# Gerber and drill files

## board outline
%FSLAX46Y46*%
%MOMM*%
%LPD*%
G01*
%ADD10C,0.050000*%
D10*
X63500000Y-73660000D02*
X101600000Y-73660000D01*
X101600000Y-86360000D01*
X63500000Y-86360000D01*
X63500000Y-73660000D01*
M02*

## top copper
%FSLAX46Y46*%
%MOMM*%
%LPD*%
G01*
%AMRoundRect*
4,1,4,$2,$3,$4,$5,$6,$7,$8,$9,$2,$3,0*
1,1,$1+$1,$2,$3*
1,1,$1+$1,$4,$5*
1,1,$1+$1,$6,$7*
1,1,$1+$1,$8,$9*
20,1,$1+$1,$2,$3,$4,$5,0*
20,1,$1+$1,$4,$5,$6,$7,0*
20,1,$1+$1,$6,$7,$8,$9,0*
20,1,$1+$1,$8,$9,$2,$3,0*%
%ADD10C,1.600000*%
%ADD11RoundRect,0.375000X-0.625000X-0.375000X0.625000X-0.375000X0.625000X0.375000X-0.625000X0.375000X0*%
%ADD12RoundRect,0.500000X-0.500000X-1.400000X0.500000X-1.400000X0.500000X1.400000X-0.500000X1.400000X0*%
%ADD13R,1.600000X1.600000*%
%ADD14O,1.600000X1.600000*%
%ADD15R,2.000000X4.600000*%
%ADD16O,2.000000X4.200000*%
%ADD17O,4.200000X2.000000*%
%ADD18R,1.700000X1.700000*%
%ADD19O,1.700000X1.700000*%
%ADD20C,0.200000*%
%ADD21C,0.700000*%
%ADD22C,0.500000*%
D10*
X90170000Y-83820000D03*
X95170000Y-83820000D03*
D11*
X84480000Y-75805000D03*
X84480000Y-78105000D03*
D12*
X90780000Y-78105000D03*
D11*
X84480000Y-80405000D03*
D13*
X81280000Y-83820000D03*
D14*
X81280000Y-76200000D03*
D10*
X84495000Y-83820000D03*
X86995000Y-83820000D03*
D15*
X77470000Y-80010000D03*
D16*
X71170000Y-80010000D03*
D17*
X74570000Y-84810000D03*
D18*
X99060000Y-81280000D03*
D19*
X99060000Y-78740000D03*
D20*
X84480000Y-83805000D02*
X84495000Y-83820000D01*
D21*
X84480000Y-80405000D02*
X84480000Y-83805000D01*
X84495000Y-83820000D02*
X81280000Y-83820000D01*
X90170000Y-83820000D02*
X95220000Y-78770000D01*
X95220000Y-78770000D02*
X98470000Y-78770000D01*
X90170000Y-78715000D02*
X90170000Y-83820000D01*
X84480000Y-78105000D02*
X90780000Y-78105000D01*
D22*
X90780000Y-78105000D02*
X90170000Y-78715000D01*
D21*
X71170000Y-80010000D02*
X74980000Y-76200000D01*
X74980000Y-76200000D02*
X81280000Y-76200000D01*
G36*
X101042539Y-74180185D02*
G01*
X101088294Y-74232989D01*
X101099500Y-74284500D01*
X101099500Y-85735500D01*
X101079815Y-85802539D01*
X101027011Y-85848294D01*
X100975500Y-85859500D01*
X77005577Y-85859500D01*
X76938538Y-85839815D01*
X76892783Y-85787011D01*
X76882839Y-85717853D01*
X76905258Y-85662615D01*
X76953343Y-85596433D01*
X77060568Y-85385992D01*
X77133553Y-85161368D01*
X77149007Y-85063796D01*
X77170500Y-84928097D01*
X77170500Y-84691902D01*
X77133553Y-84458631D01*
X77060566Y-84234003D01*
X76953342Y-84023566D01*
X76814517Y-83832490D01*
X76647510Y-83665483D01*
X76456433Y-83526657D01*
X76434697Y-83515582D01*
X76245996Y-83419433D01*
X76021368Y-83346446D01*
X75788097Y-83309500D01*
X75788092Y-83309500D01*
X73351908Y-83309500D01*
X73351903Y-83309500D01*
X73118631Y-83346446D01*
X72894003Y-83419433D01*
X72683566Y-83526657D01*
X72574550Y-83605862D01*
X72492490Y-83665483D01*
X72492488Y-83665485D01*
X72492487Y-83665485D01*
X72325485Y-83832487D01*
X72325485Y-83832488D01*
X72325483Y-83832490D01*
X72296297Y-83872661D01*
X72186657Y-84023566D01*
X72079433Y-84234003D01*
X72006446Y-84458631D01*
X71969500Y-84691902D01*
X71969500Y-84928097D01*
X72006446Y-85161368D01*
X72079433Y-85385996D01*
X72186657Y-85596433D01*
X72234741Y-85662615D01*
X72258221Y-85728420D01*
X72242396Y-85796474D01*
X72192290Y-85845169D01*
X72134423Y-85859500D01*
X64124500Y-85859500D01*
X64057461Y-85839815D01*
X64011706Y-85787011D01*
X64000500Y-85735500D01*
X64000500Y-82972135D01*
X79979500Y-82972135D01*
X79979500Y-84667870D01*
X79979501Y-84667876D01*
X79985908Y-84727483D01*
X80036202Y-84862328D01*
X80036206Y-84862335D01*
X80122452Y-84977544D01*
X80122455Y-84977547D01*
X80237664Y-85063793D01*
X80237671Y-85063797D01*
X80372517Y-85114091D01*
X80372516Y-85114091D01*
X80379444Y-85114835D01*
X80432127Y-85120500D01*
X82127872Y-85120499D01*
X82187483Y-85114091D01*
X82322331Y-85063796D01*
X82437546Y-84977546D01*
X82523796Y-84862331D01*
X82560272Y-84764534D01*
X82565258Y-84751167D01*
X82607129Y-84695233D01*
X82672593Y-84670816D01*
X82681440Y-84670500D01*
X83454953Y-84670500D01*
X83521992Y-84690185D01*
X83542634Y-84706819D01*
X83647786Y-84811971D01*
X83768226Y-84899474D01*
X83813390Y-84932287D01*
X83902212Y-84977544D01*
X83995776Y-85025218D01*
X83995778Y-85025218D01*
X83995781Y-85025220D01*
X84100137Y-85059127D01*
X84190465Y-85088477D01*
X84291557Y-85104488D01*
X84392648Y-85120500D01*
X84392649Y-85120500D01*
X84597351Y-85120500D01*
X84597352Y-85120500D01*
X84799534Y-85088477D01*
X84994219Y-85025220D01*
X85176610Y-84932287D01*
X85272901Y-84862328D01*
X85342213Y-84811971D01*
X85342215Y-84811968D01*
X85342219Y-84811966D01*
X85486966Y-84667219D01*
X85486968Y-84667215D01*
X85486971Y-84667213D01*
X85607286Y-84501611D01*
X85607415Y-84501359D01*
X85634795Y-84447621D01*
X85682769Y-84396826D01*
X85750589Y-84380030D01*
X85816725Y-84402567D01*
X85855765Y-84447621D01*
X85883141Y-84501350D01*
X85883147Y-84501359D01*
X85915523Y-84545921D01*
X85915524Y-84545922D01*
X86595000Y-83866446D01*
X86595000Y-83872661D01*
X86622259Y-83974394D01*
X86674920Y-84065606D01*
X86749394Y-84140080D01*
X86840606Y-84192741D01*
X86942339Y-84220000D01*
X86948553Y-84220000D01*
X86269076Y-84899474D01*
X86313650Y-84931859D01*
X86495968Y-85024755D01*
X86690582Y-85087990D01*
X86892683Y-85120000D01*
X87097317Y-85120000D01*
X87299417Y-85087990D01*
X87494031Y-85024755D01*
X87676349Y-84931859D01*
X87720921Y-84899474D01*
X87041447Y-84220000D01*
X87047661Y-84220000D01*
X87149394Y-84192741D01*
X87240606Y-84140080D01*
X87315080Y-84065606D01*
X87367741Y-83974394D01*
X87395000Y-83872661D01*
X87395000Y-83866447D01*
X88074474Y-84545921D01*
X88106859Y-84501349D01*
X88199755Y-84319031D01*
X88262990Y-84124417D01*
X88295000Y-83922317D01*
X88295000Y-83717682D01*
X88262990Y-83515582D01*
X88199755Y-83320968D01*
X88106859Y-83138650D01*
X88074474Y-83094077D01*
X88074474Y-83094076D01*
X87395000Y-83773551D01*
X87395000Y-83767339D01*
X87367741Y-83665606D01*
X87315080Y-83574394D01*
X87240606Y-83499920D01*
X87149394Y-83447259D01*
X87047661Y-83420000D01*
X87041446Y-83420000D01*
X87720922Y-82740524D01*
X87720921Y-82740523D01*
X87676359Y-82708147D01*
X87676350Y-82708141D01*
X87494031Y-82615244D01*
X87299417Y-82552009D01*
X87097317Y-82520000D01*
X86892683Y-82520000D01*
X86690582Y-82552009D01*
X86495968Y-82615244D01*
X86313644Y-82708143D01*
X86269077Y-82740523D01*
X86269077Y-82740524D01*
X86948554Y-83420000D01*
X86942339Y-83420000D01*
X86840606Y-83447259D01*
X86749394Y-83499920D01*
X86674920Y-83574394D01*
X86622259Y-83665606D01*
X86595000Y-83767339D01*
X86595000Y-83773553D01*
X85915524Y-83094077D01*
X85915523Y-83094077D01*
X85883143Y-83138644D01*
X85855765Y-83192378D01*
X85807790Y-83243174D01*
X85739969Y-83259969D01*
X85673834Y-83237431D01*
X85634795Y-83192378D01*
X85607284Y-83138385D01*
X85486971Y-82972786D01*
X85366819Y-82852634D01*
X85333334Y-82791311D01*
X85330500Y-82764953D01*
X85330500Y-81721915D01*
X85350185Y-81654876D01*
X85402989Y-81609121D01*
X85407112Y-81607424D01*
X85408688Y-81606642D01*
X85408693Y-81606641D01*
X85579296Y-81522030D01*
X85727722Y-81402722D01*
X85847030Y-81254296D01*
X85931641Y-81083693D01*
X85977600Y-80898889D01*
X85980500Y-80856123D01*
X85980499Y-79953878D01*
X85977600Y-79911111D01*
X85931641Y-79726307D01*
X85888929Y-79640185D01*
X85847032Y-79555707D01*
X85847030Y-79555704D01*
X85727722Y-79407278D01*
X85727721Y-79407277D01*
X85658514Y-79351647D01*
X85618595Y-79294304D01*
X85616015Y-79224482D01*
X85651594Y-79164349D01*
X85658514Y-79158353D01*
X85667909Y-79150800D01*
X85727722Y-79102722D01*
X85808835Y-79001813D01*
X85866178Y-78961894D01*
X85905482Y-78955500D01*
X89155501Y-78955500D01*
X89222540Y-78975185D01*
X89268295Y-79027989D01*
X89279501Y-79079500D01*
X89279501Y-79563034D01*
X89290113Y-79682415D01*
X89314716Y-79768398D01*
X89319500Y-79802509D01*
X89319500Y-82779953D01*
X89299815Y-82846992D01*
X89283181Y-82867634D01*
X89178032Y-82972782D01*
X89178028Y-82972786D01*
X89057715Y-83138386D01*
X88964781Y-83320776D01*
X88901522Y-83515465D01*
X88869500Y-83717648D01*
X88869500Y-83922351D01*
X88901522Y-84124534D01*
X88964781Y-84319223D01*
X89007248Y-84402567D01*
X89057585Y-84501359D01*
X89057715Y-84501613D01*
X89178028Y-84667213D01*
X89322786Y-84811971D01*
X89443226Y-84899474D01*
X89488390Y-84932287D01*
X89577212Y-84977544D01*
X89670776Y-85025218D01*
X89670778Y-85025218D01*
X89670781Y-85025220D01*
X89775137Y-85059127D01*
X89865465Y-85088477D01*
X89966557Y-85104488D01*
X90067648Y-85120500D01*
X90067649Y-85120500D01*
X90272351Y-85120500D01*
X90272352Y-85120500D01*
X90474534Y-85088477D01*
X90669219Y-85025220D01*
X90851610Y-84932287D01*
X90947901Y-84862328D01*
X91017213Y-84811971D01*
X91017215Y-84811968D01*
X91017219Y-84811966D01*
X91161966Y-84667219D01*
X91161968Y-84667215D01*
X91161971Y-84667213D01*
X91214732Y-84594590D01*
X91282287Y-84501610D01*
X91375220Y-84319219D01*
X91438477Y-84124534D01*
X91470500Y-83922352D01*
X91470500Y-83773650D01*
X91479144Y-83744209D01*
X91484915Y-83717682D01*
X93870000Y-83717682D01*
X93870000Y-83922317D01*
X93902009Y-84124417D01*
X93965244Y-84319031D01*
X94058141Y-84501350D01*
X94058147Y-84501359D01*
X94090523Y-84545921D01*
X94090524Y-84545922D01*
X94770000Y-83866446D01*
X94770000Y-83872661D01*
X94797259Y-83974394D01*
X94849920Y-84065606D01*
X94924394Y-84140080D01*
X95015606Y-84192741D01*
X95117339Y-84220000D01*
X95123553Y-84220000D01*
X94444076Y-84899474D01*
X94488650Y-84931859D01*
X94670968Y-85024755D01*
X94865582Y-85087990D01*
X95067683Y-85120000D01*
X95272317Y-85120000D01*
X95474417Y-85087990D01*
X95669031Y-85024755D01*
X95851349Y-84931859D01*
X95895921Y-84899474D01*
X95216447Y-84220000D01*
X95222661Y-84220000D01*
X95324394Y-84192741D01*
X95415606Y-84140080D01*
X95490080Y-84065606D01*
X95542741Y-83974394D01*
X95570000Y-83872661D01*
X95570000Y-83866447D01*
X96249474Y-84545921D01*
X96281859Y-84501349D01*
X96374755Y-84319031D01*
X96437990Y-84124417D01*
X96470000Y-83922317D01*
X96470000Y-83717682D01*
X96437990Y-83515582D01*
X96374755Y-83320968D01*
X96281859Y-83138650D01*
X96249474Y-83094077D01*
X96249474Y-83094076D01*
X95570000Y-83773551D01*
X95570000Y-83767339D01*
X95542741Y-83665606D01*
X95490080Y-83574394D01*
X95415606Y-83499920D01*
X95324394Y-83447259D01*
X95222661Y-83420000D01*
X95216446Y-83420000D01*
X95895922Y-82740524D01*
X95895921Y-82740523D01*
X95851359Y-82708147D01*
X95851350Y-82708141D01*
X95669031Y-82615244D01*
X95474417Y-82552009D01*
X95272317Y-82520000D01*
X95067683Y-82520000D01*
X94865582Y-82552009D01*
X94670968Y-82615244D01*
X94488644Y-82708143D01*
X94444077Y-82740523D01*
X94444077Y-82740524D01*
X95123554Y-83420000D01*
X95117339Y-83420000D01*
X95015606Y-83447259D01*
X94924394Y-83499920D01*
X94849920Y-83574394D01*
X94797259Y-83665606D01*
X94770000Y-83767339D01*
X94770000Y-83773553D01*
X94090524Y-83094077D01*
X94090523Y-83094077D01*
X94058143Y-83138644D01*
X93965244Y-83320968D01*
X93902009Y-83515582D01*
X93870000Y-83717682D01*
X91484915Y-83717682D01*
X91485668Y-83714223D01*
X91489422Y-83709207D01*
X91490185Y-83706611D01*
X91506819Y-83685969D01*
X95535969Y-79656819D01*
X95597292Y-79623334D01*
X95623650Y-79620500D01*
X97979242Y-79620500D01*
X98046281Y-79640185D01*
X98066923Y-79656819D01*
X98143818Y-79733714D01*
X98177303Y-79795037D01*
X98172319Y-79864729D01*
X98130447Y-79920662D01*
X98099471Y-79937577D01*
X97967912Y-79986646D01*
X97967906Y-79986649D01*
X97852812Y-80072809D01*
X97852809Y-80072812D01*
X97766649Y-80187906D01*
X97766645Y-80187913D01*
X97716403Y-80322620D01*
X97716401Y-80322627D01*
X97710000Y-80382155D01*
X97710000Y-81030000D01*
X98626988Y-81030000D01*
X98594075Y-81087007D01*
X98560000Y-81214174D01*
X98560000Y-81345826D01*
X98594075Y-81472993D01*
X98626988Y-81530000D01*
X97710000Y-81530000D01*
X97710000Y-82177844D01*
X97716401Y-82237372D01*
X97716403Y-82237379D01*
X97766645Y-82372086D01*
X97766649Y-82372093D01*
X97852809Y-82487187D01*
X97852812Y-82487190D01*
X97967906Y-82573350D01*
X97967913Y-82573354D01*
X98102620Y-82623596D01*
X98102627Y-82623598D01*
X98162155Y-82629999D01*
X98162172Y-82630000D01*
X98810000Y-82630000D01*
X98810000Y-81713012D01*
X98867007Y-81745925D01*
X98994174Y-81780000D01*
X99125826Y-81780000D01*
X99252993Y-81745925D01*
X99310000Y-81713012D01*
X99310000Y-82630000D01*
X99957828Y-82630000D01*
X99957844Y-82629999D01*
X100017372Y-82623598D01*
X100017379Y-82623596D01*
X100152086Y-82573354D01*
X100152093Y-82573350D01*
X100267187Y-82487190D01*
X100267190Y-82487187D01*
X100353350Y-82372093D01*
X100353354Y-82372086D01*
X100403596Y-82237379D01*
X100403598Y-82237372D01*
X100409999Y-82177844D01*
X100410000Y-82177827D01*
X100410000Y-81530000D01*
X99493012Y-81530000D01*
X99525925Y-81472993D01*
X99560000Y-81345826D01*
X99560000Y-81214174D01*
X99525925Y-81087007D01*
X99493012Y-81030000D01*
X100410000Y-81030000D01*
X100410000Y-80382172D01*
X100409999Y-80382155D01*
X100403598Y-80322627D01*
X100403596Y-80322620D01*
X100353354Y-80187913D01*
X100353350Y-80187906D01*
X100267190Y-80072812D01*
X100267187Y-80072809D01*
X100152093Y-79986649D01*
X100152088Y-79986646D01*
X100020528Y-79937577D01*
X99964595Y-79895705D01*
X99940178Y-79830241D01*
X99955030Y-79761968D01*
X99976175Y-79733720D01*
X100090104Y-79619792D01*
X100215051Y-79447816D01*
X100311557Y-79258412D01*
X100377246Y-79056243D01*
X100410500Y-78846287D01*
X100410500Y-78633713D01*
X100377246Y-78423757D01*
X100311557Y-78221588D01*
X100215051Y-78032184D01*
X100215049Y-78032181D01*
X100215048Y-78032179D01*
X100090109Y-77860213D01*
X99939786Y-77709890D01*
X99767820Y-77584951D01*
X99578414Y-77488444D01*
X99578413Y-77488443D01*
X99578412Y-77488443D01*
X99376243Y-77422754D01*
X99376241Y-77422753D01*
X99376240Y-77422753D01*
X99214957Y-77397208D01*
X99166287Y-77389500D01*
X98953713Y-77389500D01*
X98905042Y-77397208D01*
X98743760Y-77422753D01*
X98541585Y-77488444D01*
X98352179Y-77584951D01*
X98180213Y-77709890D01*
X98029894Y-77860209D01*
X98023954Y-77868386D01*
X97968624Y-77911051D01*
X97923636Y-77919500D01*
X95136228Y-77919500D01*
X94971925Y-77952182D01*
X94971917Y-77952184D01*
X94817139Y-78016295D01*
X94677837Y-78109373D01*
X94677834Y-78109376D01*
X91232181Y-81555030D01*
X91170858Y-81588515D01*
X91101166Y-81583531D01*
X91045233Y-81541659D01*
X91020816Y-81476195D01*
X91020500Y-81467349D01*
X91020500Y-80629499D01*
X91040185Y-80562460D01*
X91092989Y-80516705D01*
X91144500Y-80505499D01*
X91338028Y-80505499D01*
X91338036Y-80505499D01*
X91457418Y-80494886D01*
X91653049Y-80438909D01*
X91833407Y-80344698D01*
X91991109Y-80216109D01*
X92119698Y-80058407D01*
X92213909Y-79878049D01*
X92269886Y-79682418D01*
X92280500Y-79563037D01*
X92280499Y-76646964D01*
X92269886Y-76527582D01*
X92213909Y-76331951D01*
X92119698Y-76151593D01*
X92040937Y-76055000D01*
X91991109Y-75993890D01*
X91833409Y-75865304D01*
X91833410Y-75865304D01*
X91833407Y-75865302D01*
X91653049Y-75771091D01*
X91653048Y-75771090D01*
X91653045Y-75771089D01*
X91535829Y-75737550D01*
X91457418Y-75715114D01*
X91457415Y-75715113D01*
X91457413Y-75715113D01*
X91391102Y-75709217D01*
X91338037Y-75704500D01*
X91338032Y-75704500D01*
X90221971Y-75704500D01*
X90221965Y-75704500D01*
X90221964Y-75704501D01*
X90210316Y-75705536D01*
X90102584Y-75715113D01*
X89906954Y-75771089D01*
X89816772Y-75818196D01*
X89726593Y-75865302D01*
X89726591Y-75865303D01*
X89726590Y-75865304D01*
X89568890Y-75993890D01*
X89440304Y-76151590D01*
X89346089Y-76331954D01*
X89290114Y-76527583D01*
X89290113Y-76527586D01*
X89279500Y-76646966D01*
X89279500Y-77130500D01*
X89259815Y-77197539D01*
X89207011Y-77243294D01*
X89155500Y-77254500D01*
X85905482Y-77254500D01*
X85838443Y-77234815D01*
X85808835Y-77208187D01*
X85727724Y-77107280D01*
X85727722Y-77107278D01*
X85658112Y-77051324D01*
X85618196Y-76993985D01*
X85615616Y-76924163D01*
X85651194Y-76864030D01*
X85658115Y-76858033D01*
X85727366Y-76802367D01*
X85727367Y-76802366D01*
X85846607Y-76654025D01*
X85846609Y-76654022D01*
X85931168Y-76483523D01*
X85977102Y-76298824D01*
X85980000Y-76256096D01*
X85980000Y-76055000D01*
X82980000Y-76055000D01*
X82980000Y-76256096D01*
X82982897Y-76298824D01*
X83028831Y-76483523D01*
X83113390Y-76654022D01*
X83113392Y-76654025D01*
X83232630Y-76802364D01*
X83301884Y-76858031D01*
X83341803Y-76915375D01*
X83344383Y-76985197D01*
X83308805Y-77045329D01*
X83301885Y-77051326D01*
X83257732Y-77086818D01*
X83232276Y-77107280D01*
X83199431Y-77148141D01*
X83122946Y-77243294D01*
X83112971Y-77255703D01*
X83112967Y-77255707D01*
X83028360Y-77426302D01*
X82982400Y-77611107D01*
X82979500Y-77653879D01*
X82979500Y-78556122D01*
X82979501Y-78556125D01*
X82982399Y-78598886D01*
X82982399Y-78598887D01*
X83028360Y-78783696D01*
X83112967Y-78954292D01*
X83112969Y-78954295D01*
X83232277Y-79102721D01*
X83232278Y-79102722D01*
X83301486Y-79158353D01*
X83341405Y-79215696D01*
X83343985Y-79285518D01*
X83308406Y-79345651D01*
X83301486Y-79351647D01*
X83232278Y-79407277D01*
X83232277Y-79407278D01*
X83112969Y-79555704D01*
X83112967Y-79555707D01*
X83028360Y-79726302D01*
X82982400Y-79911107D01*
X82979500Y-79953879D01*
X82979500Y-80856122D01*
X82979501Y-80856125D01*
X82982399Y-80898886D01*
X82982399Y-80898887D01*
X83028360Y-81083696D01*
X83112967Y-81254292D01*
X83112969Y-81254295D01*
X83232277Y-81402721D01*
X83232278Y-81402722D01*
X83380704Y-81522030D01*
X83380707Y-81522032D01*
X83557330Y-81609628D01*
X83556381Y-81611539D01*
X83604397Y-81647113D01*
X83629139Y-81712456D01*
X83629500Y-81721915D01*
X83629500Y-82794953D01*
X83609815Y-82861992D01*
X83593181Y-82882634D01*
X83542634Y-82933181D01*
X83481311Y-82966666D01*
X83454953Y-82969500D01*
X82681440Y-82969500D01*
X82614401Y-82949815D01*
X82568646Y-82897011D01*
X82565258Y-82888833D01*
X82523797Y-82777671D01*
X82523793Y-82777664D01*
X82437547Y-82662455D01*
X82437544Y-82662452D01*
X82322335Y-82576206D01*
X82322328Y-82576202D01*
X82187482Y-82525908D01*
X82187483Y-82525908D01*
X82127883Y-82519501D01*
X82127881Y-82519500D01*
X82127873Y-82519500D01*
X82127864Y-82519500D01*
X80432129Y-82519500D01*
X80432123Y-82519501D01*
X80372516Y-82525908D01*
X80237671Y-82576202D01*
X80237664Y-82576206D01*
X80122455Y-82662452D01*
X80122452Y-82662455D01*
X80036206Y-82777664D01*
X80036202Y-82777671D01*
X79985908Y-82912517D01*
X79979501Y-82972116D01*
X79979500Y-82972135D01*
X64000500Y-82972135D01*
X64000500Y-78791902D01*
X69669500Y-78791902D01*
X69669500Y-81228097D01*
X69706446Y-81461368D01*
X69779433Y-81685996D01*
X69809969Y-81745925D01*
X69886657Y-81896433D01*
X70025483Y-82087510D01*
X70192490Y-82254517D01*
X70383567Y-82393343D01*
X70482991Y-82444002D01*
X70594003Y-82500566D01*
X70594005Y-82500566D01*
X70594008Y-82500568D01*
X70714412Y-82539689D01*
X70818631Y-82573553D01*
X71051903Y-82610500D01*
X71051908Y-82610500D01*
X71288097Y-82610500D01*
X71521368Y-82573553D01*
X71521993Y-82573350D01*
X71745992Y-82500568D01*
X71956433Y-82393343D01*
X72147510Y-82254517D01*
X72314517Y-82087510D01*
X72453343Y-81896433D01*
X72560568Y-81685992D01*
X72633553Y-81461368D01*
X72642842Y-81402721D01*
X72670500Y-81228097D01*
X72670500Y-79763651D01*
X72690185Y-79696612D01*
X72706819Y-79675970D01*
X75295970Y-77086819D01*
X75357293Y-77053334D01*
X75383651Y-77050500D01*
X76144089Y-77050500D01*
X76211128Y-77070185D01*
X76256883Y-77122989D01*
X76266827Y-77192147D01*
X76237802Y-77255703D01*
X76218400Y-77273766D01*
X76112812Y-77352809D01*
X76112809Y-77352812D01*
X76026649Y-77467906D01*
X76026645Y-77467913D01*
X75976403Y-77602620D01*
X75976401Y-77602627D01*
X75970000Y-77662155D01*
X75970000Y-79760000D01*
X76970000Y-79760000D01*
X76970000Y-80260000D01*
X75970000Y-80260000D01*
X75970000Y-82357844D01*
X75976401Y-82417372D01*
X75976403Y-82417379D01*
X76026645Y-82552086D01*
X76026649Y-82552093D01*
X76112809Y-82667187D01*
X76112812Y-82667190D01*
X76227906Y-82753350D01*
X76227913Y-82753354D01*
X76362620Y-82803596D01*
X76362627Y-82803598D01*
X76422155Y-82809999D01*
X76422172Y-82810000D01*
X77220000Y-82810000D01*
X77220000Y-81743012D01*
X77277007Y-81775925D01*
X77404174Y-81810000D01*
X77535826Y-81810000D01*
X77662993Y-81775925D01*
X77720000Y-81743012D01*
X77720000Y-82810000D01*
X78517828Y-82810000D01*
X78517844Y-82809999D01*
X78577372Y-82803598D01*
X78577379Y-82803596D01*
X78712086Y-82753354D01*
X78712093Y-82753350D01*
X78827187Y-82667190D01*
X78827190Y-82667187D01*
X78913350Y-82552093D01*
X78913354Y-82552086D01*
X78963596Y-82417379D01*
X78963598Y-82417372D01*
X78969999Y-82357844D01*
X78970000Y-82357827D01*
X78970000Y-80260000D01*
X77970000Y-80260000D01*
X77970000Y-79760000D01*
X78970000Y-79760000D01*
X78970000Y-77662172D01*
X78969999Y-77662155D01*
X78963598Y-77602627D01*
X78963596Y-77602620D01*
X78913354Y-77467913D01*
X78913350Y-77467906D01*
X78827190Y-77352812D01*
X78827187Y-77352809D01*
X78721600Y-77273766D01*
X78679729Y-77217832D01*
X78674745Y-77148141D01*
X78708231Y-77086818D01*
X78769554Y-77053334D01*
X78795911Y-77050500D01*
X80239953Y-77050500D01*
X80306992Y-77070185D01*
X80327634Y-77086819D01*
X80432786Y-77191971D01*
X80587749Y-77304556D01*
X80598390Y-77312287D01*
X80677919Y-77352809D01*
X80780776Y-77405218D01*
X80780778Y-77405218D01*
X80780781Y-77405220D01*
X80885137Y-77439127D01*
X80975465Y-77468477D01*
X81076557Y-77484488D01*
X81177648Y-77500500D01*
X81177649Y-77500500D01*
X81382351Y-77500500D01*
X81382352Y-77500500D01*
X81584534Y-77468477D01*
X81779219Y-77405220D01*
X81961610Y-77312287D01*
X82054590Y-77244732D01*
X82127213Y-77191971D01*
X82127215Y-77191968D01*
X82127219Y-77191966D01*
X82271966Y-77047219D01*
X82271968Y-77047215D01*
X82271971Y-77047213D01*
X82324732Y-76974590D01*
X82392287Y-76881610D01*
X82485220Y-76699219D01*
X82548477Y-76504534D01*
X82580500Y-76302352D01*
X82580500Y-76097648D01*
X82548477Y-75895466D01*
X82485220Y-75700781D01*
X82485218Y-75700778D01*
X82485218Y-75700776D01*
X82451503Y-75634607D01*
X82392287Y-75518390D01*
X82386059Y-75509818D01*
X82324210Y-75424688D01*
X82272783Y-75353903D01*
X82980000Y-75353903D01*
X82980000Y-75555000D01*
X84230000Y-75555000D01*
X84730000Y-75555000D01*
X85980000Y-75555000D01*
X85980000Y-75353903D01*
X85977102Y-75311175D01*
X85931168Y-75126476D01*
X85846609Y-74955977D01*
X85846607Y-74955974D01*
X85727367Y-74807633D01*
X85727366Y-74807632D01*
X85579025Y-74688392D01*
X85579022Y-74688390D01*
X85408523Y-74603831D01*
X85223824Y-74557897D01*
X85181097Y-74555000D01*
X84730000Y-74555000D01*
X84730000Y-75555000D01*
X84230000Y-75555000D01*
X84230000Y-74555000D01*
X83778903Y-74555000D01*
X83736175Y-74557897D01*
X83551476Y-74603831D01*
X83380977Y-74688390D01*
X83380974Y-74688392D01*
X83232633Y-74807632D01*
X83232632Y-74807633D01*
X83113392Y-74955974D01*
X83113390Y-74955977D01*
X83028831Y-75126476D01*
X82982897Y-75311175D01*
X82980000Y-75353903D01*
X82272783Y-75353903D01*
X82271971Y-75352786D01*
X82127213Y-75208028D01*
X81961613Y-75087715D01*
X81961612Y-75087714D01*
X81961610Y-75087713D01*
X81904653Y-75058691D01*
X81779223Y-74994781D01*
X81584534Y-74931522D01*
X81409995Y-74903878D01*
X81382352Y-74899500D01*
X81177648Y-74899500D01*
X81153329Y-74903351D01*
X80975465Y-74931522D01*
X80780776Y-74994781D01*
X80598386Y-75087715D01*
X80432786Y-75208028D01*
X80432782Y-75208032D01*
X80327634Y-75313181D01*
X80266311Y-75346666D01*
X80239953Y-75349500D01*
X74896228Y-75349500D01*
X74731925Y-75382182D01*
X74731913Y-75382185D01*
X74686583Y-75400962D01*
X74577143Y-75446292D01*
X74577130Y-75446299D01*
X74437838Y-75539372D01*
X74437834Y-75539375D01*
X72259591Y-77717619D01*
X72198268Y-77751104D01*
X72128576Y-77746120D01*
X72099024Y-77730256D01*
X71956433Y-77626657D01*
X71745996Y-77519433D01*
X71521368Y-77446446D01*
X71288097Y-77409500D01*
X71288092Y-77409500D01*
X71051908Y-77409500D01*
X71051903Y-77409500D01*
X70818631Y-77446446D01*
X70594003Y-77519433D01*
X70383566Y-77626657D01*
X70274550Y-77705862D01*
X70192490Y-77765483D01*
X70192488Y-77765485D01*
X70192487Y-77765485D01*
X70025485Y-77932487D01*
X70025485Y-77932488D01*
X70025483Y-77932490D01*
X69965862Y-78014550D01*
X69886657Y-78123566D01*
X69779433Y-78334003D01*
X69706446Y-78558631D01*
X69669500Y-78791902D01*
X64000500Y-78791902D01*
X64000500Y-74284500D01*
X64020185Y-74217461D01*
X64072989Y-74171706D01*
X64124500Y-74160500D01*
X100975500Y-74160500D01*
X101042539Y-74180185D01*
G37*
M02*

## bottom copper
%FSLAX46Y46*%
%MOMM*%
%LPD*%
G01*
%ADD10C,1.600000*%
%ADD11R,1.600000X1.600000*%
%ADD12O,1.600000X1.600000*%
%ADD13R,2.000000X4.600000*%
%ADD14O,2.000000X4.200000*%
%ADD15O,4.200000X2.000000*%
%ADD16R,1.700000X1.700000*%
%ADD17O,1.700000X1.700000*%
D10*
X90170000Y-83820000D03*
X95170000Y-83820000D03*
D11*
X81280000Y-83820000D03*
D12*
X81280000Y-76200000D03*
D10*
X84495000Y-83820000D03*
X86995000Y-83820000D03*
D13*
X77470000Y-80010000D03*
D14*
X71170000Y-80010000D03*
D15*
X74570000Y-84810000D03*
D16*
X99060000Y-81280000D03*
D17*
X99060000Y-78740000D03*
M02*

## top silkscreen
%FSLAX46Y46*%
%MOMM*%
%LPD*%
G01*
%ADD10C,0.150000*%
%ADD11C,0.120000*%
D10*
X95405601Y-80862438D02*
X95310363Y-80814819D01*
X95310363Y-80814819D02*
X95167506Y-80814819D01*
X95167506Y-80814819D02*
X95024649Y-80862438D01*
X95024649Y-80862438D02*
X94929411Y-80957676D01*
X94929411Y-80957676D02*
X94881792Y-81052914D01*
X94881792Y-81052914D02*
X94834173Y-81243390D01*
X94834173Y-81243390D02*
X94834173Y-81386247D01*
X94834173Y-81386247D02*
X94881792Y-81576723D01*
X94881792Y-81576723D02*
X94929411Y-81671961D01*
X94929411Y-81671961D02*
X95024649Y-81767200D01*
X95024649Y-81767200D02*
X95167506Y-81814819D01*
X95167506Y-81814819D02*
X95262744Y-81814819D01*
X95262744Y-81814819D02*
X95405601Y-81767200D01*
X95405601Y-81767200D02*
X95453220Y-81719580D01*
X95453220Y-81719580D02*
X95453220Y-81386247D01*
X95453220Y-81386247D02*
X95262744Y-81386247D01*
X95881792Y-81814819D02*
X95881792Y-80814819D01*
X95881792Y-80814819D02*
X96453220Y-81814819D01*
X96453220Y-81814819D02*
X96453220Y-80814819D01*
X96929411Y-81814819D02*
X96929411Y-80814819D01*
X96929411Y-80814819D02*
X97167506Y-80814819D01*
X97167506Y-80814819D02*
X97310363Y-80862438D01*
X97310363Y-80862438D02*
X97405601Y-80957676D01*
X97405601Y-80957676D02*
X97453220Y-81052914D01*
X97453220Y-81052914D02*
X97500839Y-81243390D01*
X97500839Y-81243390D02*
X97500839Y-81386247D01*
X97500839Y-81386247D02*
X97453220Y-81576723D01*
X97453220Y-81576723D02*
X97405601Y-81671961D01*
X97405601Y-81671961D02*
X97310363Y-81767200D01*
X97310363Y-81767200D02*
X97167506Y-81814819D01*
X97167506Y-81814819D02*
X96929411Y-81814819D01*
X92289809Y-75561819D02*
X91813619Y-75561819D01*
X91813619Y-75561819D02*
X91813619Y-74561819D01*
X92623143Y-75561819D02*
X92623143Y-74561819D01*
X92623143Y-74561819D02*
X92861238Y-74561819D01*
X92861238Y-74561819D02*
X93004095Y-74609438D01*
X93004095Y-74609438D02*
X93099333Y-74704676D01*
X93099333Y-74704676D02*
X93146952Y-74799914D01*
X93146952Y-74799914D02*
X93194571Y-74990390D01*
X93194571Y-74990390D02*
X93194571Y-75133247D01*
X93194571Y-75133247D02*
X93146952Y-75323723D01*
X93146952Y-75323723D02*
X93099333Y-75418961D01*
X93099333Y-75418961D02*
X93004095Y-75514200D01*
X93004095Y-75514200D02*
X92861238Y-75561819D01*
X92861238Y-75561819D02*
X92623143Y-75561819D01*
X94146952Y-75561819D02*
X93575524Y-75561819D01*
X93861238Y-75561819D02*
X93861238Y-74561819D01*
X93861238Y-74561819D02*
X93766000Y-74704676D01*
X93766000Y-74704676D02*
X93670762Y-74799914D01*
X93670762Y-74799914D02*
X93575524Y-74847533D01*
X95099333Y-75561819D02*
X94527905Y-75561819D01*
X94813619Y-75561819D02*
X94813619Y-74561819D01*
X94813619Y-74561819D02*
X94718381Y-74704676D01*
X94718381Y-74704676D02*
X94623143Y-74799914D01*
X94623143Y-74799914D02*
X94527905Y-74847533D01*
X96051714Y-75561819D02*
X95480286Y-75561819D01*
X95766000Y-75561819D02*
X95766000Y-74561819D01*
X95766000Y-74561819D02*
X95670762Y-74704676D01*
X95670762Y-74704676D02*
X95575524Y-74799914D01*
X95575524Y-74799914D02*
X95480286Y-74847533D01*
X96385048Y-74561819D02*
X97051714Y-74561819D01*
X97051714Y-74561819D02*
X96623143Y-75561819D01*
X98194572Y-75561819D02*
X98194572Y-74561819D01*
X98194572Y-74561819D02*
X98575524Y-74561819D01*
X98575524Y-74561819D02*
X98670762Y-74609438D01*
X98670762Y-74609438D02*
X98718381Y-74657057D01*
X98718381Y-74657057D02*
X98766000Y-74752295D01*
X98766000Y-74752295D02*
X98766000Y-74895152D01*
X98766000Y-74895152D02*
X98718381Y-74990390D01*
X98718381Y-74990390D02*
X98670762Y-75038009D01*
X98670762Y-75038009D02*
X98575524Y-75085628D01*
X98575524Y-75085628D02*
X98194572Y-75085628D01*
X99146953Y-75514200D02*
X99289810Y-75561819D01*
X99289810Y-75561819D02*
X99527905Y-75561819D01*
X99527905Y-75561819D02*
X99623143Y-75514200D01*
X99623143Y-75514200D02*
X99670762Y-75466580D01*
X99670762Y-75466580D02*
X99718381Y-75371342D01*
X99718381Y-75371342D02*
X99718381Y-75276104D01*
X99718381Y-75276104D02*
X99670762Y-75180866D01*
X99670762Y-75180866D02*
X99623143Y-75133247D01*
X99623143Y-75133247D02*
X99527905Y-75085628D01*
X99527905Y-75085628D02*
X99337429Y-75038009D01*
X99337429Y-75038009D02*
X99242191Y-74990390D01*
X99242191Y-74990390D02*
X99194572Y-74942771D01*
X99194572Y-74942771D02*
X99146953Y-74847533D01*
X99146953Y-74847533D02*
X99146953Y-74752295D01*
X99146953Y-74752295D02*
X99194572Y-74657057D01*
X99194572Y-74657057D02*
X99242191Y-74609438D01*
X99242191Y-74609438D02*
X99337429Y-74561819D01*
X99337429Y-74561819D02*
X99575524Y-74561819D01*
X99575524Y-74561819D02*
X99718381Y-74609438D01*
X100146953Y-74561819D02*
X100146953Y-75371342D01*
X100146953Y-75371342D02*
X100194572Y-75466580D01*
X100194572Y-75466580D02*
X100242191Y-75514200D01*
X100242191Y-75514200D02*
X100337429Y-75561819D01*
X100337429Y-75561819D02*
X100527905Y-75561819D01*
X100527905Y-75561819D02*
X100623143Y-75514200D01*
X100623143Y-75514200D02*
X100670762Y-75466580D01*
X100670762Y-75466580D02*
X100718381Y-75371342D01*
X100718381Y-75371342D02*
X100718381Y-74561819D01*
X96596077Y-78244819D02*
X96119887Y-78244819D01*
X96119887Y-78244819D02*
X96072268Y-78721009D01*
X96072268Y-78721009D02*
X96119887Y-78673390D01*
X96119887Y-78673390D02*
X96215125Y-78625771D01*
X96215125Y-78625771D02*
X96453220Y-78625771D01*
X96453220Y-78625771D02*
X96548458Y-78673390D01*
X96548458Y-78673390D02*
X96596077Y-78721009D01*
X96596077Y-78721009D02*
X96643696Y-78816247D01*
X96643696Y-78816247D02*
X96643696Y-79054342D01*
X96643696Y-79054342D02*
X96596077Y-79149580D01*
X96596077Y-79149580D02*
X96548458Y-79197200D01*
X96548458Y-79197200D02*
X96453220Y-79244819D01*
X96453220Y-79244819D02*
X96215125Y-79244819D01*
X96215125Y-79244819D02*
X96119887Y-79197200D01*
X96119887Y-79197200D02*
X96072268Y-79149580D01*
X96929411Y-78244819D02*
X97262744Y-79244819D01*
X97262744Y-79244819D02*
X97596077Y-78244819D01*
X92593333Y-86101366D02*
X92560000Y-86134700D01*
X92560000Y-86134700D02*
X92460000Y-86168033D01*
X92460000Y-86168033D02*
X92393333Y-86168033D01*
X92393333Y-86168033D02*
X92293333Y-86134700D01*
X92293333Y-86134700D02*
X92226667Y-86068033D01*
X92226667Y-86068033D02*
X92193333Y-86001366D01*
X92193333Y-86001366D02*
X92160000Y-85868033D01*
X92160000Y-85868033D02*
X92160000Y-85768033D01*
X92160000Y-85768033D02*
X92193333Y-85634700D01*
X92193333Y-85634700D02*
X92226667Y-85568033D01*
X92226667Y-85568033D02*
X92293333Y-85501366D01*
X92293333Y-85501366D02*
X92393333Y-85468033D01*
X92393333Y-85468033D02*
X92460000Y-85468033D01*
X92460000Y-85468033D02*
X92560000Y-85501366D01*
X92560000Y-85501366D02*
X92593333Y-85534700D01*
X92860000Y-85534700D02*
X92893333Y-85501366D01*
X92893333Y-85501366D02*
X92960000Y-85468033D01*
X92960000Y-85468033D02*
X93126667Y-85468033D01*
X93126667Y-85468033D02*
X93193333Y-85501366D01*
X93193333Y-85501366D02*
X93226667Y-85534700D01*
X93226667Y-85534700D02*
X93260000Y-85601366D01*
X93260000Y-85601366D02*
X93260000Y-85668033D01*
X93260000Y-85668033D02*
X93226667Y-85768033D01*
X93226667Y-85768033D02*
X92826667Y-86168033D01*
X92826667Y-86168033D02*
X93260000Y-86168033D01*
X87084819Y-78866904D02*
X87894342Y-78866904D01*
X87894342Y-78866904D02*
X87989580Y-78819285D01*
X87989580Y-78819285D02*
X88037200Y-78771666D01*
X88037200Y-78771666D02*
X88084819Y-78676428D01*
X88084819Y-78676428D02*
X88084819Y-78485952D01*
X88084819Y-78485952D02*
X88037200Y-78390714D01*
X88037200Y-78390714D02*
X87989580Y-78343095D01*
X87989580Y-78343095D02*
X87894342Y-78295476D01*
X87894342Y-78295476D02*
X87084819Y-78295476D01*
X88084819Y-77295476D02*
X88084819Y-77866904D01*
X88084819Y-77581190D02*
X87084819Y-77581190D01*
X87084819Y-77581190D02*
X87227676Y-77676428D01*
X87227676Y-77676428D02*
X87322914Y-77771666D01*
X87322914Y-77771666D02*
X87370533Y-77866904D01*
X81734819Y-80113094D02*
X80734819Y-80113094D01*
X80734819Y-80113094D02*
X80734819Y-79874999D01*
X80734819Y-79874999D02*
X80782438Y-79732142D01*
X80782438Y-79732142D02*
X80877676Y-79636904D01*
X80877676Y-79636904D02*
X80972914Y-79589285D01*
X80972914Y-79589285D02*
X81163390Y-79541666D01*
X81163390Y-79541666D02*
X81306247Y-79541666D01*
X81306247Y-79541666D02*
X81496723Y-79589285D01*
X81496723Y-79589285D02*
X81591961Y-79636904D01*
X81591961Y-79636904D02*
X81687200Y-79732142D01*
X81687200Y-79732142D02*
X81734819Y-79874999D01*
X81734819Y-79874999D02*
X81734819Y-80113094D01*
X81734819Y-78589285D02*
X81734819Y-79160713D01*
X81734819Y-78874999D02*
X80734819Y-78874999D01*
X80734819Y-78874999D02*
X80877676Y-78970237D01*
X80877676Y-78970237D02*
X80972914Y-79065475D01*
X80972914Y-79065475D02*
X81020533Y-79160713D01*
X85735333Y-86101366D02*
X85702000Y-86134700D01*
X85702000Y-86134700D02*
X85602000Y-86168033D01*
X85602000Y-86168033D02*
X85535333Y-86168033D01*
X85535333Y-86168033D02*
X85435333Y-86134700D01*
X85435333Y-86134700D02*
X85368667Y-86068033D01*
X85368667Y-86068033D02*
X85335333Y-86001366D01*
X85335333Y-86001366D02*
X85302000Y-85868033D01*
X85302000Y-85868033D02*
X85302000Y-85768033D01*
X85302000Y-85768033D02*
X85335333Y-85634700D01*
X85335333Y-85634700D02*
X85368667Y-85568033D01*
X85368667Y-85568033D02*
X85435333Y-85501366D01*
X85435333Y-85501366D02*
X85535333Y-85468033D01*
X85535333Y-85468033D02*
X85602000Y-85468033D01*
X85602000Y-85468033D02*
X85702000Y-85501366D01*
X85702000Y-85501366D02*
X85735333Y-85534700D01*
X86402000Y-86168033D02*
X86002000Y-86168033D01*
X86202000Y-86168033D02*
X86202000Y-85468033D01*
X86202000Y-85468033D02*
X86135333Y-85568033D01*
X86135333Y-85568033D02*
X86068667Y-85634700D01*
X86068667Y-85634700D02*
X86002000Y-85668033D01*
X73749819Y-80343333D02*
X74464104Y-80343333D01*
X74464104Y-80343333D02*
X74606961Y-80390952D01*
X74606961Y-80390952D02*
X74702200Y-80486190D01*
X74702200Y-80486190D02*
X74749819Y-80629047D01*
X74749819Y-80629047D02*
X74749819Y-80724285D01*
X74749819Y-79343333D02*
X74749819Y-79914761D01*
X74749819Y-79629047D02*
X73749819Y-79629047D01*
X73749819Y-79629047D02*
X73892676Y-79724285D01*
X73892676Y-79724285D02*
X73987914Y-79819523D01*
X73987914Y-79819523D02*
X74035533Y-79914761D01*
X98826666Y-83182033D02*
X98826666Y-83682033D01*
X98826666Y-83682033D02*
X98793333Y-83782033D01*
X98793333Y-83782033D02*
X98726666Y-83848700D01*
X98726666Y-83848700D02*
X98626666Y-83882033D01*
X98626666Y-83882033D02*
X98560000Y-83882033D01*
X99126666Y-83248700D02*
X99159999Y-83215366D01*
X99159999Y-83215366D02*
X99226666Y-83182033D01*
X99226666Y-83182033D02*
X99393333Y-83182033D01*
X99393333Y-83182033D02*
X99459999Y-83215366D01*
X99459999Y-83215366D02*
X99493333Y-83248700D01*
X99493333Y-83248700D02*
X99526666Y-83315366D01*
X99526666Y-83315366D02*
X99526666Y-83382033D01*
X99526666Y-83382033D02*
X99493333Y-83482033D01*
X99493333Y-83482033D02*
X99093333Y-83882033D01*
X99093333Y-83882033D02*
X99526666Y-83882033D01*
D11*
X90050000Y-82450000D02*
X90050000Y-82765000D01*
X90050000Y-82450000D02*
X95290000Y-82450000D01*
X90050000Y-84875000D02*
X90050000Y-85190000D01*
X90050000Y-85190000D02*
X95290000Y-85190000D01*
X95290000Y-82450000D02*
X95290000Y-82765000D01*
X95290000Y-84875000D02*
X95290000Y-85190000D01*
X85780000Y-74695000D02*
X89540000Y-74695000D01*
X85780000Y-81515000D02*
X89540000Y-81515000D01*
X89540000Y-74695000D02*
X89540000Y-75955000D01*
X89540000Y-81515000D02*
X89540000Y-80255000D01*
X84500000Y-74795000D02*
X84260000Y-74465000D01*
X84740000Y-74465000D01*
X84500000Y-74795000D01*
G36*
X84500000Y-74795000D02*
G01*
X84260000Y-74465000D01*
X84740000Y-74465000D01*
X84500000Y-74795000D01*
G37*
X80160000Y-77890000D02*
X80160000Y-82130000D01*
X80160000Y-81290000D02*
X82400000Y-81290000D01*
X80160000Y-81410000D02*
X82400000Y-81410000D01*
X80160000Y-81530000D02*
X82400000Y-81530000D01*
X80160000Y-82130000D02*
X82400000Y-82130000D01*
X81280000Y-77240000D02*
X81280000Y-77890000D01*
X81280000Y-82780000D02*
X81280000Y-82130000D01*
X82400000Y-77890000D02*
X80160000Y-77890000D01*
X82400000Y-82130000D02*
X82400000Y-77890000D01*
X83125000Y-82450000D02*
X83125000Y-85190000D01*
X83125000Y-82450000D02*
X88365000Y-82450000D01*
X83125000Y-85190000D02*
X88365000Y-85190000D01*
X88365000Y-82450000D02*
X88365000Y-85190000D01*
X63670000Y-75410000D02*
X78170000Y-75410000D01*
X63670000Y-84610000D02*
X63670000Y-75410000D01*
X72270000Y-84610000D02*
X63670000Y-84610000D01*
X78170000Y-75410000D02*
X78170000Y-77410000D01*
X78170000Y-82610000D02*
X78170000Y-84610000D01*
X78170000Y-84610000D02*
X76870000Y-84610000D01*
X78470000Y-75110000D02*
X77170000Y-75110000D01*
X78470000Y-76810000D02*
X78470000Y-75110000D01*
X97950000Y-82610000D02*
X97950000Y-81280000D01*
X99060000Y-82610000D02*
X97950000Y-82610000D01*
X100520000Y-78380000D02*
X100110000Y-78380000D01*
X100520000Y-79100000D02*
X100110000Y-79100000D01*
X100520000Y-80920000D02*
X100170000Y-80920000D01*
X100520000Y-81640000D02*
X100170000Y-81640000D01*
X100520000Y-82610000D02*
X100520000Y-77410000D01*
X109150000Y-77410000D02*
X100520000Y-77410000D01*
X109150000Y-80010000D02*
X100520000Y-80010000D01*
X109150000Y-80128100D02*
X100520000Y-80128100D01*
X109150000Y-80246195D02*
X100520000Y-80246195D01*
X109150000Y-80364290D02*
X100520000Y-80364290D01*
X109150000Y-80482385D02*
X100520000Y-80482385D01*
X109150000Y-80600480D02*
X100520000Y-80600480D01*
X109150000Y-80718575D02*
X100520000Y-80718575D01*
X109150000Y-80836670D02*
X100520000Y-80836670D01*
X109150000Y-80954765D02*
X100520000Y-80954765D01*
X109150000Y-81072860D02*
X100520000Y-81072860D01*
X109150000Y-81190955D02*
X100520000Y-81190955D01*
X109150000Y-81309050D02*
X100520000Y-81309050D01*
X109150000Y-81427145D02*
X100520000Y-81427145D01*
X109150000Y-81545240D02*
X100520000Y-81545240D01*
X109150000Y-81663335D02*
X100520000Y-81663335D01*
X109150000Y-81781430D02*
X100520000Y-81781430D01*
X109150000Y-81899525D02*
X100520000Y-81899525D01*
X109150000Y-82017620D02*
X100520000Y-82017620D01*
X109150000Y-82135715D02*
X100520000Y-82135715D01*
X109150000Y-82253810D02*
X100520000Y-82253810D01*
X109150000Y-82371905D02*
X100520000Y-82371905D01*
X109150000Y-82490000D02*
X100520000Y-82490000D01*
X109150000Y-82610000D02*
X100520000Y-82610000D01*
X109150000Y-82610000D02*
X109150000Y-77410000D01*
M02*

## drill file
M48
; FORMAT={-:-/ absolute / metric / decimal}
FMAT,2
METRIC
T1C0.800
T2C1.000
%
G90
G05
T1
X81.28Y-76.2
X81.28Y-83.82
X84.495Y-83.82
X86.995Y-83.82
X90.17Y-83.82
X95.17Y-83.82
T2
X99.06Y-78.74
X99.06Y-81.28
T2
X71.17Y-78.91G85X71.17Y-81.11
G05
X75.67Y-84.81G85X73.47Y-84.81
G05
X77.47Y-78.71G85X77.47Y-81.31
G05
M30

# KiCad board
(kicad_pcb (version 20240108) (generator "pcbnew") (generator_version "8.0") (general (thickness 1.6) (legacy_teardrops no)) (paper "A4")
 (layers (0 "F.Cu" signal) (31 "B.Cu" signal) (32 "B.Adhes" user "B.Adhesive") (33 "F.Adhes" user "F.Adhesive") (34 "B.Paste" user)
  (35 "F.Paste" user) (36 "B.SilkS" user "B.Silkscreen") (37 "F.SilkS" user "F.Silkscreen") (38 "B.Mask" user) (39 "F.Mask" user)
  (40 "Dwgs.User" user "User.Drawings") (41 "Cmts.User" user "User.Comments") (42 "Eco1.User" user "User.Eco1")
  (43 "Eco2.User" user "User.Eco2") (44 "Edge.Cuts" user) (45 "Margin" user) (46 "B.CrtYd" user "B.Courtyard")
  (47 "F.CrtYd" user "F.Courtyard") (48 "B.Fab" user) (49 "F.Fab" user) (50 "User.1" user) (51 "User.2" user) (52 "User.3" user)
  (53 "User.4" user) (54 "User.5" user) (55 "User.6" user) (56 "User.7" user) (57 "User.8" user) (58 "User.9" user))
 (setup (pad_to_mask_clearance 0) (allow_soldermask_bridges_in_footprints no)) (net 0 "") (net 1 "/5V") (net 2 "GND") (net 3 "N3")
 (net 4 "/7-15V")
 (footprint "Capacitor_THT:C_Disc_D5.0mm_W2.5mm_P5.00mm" (layer "F.Cu") (at 90.17 83.82)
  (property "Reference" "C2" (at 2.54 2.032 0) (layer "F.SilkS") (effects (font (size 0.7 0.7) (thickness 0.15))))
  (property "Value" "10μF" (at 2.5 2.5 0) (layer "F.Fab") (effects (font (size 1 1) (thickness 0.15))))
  (fp_line (start -0.12 -1.37) (end -0.12 -1.055) (stroke (width 0.12) (type solid)) (layer "F.SilkS"))
  (fp_line (start -0.12 -1.37) (end 5.12 -1.37) (stroke (width 0.12) (type solid)) (layer "F.SilkS"))
  (fp_line (start -0.12 1.055) (end -0.12 1.37) (stroke (width 0.12) (type solid)) (layer "F.SilkS"))
  (fp_line (start -0.12 1.37) (end 5.12 1.37) (stroke (width 0.12) (type solid)) (layer "F.SilkS"))
  (fp_line (start 5.12 -1.37) (end 5.12 -1.055) (stroke (width 0.12) (type solid)) (layer "F.SilkS"))
  (fp_line (start 5.12 1.055) (end 5.12 1.37) (stroke (width 0.12) (type solid)) (layer "F.SilkS"))
  (pad "1" thru_hole circle (at 0 0) (size 1.6 1.6) (drill 0.8) (layers "*.Cu" "*.Mask") (remove_unused_layers no) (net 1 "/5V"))
  (pad "2" thru_hole circle (at 5 0) (size 1.6 1.6) (drill 0.8) (layers "*.Cu" "*.Mask") (remove_unused_layers no) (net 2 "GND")))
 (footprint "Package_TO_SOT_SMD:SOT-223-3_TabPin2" (layer "F.Cu") (at 87.63 78.105)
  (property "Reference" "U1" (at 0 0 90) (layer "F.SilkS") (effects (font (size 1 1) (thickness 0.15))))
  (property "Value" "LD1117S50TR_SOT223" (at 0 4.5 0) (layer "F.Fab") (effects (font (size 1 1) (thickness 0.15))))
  (fp_line (start -1.85 -3.41) (end 1.91 -3.41) (stroke (width 0.12) (type solid)) (layer "F.SilkS"))
  (fp_line (start -1.85 3.41) (end 1.91 3.41) (stroke (width 0.12) (type solid)) (layer "F.SilkS"))
  (fp_line (start 1.91 -3.41) (end 1.91 -2.15) (stroke (width 0.12) (type solid)) (layer "F.SilkS"))
  (fp_line (start 1.91 3.41) (end 1.91 2.15) (stroke (width 0.12) (type solid)) (layer "F.SilkS"))
  (fp_poly
   (pts (xy -3.13 -3.31) (xy -3.37 -3.64) (xy -2.89 -3.64) (xy -3.13 -3.31)) (stroke (width 0.12) (type solid)) (fill solid)
   (layer "F.SilkS"))
  (pad "1" smd roundrect (at -3.15 -2.3) (size 2 1.5) (layers "F.Cu" "F.Paste" "F.Mask") (roundrect_rratio 0.25) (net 2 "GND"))
  (pad "2" smd roundrect (at -3.15 0) (size 2 1.5) (layers "F.Cu" "F.Paste" "F.Mask") (roundrect_rratio 0.25) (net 1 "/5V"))
  (pad "2" smd roundrect (at 3.15 0) (size 2 3.8) (layers "F.Cu" "F.Paste" "F.Mask") (roundrect_rratio 0.25) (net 1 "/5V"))
  (pad "3" smd roundrect (at -3.15 2.3) (size 2 1.5) (layers "F.Cu" "F.Paste" "F.Mask") (roundrect_rratio 0.25) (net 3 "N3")))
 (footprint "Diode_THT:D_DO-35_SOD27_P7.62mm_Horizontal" (layer "F.Cu") (at 81.28 83.82 90)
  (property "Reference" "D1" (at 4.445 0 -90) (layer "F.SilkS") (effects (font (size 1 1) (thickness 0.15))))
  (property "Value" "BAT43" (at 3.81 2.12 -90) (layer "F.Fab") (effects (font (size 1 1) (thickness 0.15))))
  (fp_line (start 5.93 -1.12) (end 1.69 -1.12) (stroke (width 0.12) (type solid)) (layer "F.SilkS"))
  (fp_line (start 2.53 -1.12) (end 2.53 1.12) (stroke (width 0.12) (type solid)) (layer "F.SilkS"))
  (fp_line (start 2.41 -1.12) (end 2.41 1.12) (stroke (width 0.12) (type solid)) (layer "F.SilkS"))
  (fp_line (start 2.29 -1.12) (end 2.29 1.12) (stroke (width 0.12) (type solid)) (layer "F.SilkS"))
  (fp_line (start 1.69 -1.12) (end 1.69 1.12) (stroke (width 0.12) (type solid)) (layer "F.SilkS"))
  (fp_line (start 6.58 0) (end 5.93 0) (stroke (width 0.12) (type solid)) (layer "F.SilkS"))
  (fp_line (start 1.04 0) (end 1.69 0) (stroke (width 0.12) (type solid)) (layer "F.SilkS"))
  (fp_line (start 5.93 1.12) (end 5.93 -1.12) (stroke (width 0.12) (type solid)) (layer "F.SilkS"))
  (fp_line (start 1.69 1.12) (end 5.93 1.12) (stroke (width 0.12) (type solid)) (layer "F.SilkS"))
  (pad "1" thru_hole rect (at 0 0 90) (size 1.6 1.6) (drill 0.8) (layers "*.Cu" "*.Mask") (remove_unused_layers no) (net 3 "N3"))
  (pad "2" thru_hole oval (at 7.62 0 90) (size 1.6 1.6) (drill 0.8) (layers "*.Cu" "*.Mask") (remove_unused_layers no) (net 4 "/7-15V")))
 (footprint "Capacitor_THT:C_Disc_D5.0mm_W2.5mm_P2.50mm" (layer "F.Cu") (at 84.495 83.82)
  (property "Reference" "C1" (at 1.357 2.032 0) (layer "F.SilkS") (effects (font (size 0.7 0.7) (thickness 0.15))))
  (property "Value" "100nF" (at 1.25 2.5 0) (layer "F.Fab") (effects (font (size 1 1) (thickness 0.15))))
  (fp_line (start -1.37 -1.37) (end -1.37 1.37) (stroke (width 0.12) (type solid)) (layer "F.SilkS"))
  (fp_line (start -1.37 -1.37) (end 3.87 -1.37) (stroke (width 0.12) (type solid)) (layer "F.SilkS"))
  (fp_line (start -1.37 1.37) (end 3.87 1.37) (stroke (width 0.12) (type solid)) (layer "F.SilkS"))
  (fp_line (start 3.87 -1.37) (end 3.87 1.37) (stroke (width 0.12) (type solid)) (layer "F.SilkS"))
  (pad "1" thru_hole circle (at 0 0) (size 1.6 1.6) (drill 0.8) (layers "*.Cu" "*.Mask") (remove_unused_layers no) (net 3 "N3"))
  (pad "2" thru_hole circle (at 2.5 0) (size 1.6 1.6) (drill 0.8) (layers "*.Cu" "*.Mask") (remove_unused_layers no) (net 2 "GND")))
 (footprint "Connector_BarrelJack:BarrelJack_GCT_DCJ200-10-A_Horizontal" (layer "F.Cu") (at 77.47 80.01 -90)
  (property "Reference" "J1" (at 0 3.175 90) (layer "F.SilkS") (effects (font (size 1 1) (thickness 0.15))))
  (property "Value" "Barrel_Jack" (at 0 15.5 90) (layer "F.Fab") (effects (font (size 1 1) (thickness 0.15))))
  (fp_line (start -4.6 13.8) (end -4.6 -0.7) (stroke (width 0.12) (type solid)) (layer "F.SilkS"))
  (fp_line (start 4.6 13.8) (end -4.6 13.8) (stroke (width 0.12) (type solid)) (layer "F.SilkS"))
  (fp_line (start 4.6 5.2) (end 4.6 13.8) (stroke (width 0.12) (type solid)) (layer "F.SilkS"))
  (fp_line (start -4.6 -0.7) (end -2.6 -0.7) (stroke (width 0.12) (type solid)) (layer "F.SilkS"))
  (fp_line (start 2.6 -0.7) (end 4.6 -0.7) (stroke (width 0.12) (type solid)) (layer "F.SilkS"))
  (fp_line (start 4.6 -0.7) (end 4.6 0.6) (stroke (width 0.12) (type solid)) (layer "F.SilkS"))
  (fp_line (start -4.9 -1) (end -4.9 0.3) (stroke (width 0.12) (type solid)) (layer "F.SilkS"))
  (fp_line (start -3.2 -1) (end -4.9 -1) (stroke (width 0.12) (type solid)) (layer "F.SilkS"))
  (pad "1" thru_hole rect (at 0 0 270) (size 4.6 2) (drill oval 3.6 1) (layers "*.Cu" "*.Mask") (remove_unused_layers no) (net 2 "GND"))
  (pad "2" thru_hole oval (at 0 6.3 270) (size 4.2 2) (drill oval 3.2 1) (layers "*.Cu" "*.Mask") (remove_unused_layers no) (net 4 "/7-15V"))
  (pad "3" thru_hole oval (at 4.8 2.9 270) (size 2 4.2) (drill oval 1 3.2) (layers "*.Cu" "*.Mask") (remove_unused_layers no)))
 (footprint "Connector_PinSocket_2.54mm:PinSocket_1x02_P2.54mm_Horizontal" (layer "F.Cu") (at 99.06 81.28 180)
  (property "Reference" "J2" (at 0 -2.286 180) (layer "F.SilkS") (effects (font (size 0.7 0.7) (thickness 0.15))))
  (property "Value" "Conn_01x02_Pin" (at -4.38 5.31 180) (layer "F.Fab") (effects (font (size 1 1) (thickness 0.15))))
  (fp_line (start 1.11 -1.33) (end 1.11 0) (stroke (width 0.12) (type solid)) (layer "F.SilkS"))
  (fp_line (start 0 -1.33) (end 1.11 -1.33) (stroke (width 0.12) (type solid)) (layer "F.SilkS"))
  (fp_line (start -1.46 2.9) (end -1.05 2.9) (stroke (width 0.12) (type solid)) (layer "F.SilkS"))
  (fp_line (start -1.46 2.18) (end -1.05 2.18) (stroke (width 0.12) (type solid)) (layer "F.SilkS"))
  (fp_line (start -1.46 0.36) (end -1.11 0.36) (stroke (width 0.12) (type solid)) (layer "F.SilkS"))
  (fp_line (start -1.46 -0.36) (end -1.11 -0.36) (stroke (width 0.12) (type solid)) (layer "F.SilkS"))
  (fp_line (start -1.46 -1.33) (end -1.46 3.87) (stroke (width 0.12) (type solid)) (layer "F.SilkS"))
  (fp_line (start -10.09 3.87) (end -1.46 3.87) (stroke (width 0.12) (type solid)) (layer "F.SilkS"))
  (fp_line (start -10.09 1.27) (end -1.46 1.27) (stroke (width 0.12) (type solid)) (layer "F.SilkS"))
  (fp_line (start -10.09 1.1519) (end -1.46 1.1519) (stroke (width 0.12) (type solid)) (layer "F.SilkS"))
  (fp_line (start -10.09 1.033805) (end -1.46 1.033805) (stroke (width 0.12) (type solid)) (layer "F.SilkS"))
  (fp_line (start -10.09 0.91571) (end -1.46 0.91571) (stroke (width 0.12) (type solid)) (layer "F.SilkS"))
  (fp_line (start -10.09 0.797615) (end -1.46 0.797615) (stroke (width 0.12) (type solid)) (layer "F.SilkS"))
  (fp_line (start -10.09 0.67952) (end -1.46 0.67952) (stroke (width 0.12) (type solid)) (layer "F.SilkS"))
  (fp_line (start -10.09 0.561425) (end -1.46 0.561425) (stroke (width 0.12) (type solid)) (layer "F.SilkS"))
  (fp_line (start -10.09 0.44333) (end -1.46 0.44333) (stroke (width 0.12) (type solid)) (layer "F.SilkS"))
  (fp_line (start -10.09 0.325235) (end -1.46 0.325235) (stroke (width 0.12) (type solid)) (layer "F.SilkS"))
  (fp_line (start -10.09 0.20714) (end -1.46 0.20714) (stroke (width 0.12) (type solid)) (layer "F.SilkS"))
  (fp_line (start -10.09 0.089045) (end -1.46 0.089045) (stroke (width 0.12) (type solid)) (layer "F.SilkS"))
  (fp_line (start -10.09 -0.02905) (end -1.46 -0.02905) (stroke (width 0.12) (type solid)) (layer "F.SilkS"))
  (fp_line (start -10.09 -0.147145) (end -1.46 -0.147145) (stroke (width 0.12) (type solid)) (layer "F.SilkS"))
  (fp_line (start -10.09 -0.26524) (end -1.46 -0.26524) (stroke (width 0.12) (type solid)) (layer "F.SilkS"))
  (fp_line (start -10.09 -0.383335) (end -1.46 -0.383335) (stroke (width 0.12) (type solid)) (layer "F.SilkS"))
  (fp_line (start -10.09 -0.50143) (end -1.46 -0.50143) (stroke (width 0.12) (type solid)) (layer "F.SilkS"))
  (fp_line (start -10.09 -0.619525) (end -1.46 -0.619525) (stroke (width 0.12) (type solid)) (layer "F.SilkS"))
  (fp_line (start -10.09 -0.73762) (end -1.46 -0.73762) (stroke (width 0.12) (type solid)) (layer "F.SilkS"))
  (fp_line (start -10.09 -0.855715) (end -1.46 -0.855715) (stroke (width 0.12) (type solid)) (layer "F.SilkS"))
  (fp_line (start -10.09 -0.97381) (end -1.46 -0.97381) (stroke (width 0.12) (type solid)) (layer "F.SilkS"))
  (fp_line (start -10.09 -1.091905) (end -1.46 -1.091905) (stroke (width 0.12) (type solid)) (layer "F.SilkS"))
  (fp_line (start -10.09 -1.21) (end -1.46 -1.21) (stroke (width 0.12) (type solid)) (layer "F.SilkS"))
  (fp_line (start -10.09 -1.33) (end -1.46 -1.33) (stroke (width 0.12) (type solid)) (layer "F.SilkS"))
  (fp_line (start -10.09 -1.33) (end -10.09 3.87) (stroke (width 0.12) (type solid)) (layer "F.SilkS"))
  (pad "1" thru_hole rect (at 0 0 180) (size 1.7 1.7) (drill 1) (layers "*.Cu" "*.Mask") (remove_unused_layers no) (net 2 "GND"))
  (pad "2" thru_hole oval (at 0 2.54 180) (size 1.7 1.7) (drill 1) (layers "*.Cu" "*.Mask") (remove_unused_layers no) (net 1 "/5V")))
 (gr_rect (start 63.5 73.66) (end 101.6 86.36) (stroke (width 0.05) (type default)) (fill none) (layer "Edge.Cuts"))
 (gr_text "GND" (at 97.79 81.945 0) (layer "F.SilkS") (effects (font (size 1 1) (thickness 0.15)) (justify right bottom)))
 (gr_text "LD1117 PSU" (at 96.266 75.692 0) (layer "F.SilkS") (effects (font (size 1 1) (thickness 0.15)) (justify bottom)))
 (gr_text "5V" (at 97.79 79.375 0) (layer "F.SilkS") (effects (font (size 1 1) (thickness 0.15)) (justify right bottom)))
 (segment (start 84.48 83.805) (end 84.495 83.82) (width 0.2) (layer "F.Cu") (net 3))
 (segment (start 84.48 80.405) (end 84.48 83.805) (width 0.7) (layer "F.Cu") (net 3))
 (segment (start 84.495 83.82) (end 81.28 83.82) (width 0.7) (layer "F.Cu") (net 3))
 (segment (start 90.17 83.82) (end 95.22 78.77) (width 0.7) (layer "F.Cu") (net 1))
 (segment (start 95.22 78.77) (end 98.47 78.77) (width 0.7) (layer "F.Cu") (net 1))
 (segment (start 90.17 78.715) (end 90.17 83.82) (width 0.7) (layer "F.Cu") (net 1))
 (segment (start 84.48 78.105) (end 90.78 78.105) (width 0.7) (layer "F.Cu") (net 1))
 (segment (start 90.78 78.105) (end 90.17 78.715) (width 0.5) (layer "F.Cu") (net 1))
 (segment (start 71.17 80.01) (end 74.98 76.2) (width 0.7) (layer "F.Cu") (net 4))
 (segment (start 74.98 76.2) (end 81.28 76.2) (width 0.7) (layer "F.Cu") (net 4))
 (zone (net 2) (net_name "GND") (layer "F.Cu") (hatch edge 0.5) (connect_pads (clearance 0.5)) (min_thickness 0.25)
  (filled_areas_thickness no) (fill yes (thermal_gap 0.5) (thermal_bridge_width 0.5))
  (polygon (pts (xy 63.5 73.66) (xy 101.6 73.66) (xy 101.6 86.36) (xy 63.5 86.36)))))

